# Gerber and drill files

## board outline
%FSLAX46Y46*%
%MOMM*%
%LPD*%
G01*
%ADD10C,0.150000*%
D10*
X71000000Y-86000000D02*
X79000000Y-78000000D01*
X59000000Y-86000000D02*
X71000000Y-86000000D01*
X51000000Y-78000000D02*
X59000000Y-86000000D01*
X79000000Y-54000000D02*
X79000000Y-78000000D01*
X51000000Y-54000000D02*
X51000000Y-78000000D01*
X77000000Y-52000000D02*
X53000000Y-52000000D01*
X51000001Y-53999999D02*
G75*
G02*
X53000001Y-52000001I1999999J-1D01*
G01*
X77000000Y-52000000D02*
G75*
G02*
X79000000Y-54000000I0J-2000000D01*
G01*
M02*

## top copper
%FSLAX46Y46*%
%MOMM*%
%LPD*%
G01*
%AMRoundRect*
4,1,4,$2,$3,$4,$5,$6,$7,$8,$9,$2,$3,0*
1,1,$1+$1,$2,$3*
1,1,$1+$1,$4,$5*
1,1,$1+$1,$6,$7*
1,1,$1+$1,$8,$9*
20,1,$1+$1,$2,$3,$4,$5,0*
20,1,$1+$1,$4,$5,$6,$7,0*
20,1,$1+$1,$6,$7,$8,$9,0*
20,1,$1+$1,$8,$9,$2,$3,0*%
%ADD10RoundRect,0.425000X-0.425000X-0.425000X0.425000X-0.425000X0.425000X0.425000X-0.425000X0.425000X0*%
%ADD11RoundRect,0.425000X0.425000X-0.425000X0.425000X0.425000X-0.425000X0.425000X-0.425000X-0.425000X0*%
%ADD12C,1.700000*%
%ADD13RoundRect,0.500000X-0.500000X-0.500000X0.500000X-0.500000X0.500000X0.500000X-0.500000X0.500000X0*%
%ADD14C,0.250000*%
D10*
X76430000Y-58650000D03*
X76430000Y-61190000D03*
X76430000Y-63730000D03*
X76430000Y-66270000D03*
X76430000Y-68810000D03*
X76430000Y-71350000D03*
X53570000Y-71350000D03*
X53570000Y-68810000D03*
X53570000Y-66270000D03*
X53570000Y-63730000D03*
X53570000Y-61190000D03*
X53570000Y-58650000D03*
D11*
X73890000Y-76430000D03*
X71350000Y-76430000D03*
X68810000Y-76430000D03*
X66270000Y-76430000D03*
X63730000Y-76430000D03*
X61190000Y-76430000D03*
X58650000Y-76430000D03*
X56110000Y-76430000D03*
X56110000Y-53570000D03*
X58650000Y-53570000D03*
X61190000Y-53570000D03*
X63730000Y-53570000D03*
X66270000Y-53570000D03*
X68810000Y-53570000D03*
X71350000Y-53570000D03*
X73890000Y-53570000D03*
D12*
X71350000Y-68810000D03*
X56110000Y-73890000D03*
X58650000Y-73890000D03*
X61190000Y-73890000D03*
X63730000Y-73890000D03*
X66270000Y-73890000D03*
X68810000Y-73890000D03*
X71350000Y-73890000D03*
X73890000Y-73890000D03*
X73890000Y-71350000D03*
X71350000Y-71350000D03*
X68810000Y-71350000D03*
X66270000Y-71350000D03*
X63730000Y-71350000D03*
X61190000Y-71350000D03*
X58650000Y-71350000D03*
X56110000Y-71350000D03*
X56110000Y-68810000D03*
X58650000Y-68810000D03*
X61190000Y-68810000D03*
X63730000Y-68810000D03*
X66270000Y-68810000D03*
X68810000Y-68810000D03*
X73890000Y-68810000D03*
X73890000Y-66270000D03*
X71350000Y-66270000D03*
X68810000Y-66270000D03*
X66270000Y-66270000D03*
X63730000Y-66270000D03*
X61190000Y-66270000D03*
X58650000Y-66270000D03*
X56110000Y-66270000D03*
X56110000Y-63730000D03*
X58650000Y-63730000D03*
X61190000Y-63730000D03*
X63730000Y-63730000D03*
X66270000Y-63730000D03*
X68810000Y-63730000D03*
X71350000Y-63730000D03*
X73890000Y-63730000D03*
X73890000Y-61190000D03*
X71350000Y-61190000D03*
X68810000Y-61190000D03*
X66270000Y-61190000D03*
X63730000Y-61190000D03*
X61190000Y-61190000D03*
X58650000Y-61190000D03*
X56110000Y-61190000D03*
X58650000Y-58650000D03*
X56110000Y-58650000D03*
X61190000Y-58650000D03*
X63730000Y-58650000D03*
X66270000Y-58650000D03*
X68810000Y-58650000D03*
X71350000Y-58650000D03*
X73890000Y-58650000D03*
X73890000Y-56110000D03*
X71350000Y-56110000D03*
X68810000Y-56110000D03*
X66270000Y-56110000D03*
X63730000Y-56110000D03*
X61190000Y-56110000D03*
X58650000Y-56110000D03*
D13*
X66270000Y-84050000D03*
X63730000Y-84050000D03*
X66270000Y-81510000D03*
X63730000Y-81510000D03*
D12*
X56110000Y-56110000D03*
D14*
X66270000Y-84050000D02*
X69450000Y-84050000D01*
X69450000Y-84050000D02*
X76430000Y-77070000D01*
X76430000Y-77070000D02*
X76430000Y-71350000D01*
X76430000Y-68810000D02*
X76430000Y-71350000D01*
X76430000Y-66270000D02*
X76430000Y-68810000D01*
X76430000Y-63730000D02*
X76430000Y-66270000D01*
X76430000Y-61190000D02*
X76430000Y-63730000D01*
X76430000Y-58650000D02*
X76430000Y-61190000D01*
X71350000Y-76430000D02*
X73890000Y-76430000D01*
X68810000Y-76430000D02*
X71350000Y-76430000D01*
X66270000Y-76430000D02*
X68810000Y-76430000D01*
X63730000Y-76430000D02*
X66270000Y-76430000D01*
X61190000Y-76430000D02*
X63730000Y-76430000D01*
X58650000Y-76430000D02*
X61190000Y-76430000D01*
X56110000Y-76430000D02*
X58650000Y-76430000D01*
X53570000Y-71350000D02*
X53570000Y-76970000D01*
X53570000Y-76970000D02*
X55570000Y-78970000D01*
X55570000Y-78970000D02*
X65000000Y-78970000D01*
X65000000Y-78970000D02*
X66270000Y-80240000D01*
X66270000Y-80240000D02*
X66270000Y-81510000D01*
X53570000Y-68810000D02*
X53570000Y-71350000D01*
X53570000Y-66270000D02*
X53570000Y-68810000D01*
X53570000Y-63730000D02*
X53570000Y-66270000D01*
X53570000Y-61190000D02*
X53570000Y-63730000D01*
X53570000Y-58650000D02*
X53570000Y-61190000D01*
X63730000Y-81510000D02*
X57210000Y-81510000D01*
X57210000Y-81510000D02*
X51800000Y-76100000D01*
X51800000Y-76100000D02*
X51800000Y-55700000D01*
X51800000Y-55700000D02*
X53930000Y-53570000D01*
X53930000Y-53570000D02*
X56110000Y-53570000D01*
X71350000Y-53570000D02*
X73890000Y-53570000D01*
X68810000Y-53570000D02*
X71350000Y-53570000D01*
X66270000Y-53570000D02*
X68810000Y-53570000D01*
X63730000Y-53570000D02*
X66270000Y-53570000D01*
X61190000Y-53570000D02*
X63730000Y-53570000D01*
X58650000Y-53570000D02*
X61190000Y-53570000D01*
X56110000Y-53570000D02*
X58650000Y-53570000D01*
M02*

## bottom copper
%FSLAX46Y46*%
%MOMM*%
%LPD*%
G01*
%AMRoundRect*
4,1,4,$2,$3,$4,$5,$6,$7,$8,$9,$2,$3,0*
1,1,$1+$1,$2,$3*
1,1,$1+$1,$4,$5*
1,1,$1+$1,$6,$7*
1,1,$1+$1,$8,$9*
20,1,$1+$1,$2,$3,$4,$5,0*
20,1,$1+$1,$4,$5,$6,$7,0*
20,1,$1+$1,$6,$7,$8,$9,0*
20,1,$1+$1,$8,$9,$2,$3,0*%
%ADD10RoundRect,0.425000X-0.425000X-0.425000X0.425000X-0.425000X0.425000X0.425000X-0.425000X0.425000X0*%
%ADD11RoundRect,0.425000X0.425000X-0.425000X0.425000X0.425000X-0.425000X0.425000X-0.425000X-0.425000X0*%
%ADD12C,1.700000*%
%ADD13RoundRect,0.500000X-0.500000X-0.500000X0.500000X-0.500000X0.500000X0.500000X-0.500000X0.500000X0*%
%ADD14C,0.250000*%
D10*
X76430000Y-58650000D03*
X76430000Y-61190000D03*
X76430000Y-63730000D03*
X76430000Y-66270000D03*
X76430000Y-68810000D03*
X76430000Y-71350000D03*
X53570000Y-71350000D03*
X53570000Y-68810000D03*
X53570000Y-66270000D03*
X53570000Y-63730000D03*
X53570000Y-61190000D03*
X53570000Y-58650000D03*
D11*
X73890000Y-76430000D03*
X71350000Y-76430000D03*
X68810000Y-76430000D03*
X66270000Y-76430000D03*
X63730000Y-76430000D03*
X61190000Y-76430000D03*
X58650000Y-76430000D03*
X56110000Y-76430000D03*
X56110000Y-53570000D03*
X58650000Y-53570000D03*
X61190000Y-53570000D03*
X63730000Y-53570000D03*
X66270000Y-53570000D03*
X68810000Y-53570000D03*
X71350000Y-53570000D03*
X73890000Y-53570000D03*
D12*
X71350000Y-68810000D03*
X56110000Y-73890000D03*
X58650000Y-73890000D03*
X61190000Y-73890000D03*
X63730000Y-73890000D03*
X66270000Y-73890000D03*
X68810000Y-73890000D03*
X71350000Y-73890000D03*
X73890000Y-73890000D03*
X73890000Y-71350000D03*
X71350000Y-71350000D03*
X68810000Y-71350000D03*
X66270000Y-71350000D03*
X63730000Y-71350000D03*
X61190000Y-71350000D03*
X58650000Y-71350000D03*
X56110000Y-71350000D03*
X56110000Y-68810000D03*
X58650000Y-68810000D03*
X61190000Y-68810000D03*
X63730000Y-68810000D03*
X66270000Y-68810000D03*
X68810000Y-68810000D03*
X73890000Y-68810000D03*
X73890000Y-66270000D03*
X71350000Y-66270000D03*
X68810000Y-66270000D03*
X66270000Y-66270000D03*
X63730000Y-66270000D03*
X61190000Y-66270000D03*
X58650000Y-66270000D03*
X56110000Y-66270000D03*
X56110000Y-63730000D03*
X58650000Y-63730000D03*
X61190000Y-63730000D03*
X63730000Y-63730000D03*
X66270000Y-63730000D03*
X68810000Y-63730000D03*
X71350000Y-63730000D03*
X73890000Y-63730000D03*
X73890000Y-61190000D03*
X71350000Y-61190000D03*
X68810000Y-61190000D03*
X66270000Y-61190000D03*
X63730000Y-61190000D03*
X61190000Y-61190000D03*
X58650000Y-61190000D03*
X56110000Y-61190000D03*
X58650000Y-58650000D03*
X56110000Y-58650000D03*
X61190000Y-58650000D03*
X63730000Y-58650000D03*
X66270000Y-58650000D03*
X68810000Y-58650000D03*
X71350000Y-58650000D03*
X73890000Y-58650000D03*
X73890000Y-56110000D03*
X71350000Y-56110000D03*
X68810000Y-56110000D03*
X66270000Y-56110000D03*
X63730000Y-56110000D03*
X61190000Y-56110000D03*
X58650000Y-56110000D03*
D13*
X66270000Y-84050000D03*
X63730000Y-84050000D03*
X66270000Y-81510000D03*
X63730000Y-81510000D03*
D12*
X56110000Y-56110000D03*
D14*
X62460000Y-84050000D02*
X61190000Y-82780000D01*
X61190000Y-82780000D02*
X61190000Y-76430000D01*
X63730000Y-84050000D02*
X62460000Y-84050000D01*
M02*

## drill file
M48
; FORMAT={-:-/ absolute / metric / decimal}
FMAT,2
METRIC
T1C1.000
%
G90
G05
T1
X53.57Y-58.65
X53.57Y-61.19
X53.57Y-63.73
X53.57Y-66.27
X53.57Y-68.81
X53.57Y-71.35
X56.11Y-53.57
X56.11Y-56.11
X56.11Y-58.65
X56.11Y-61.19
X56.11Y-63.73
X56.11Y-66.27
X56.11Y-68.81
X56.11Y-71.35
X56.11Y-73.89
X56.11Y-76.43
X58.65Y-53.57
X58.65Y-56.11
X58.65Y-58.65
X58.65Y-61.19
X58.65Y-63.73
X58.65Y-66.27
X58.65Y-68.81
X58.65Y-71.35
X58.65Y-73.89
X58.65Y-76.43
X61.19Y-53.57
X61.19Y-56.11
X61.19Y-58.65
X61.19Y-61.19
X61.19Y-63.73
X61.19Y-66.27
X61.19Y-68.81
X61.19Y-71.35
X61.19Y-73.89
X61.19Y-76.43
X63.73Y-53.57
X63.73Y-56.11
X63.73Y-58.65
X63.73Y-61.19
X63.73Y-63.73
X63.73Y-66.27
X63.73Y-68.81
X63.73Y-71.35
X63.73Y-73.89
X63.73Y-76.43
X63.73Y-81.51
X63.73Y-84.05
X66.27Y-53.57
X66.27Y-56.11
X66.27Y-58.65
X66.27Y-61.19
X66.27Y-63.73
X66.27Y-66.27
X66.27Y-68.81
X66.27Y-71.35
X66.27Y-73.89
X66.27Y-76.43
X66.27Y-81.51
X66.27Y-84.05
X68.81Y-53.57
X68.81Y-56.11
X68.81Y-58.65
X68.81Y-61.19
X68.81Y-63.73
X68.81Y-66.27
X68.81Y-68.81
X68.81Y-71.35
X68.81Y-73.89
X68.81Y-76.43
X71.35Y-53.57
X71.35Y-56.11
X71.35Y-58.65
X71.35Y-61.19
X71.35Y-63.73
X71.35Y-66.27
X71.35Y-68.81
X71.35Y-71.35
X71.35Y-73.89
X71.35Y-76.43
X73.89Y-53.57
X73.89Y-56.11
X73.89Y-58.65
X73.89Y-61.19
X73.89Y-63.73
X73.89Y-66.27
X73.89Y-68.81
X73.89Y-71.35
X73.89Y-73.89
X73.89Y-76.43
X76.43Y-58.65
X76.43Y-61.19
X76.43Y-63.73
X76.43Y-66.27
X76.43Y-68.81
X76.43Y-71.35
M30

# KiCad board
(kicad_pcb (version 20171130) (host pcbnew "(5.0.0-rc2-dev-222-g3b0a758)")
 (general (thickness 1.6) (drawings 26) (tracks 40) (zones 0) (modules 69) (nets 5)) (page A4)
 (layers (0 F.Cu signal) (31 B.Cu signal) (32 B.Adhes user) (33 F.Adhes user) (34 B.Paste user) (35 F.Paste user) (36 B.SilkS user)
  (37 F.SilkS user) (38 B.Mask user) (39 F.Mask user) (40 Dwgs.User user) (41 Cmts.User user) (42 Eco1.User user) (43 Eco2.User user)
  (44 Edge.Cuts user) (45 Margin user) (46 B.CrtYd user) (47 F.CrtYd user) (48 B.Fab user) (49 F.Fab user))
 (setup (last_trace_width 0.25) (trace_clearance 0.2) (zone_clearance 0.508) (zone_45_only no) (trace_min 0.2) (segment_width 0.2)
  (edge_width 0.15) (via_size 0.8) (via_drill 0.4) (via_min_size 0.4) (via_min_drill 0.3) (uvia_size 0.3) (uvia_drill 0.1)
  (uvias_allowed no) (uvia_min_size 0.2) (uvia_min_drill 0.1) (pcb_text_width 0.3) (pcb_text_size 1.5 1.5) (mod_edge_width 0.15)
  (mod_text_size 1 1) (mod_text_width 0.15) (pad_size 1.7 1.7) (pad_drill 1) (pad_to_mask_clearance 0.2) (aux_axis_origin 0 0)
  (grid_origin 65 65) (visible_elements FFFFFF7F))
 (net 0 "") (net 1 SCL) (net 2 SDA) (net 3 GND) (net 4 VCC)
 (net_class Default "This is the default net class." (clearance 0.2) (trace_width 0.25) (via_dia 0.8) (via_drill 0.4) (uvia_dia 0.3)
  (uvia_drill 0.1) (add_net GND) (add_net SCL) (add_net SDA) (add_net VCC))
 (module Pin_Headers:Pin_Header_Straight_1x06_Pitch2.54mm (layer F.Cu) (at 76.43 58.65)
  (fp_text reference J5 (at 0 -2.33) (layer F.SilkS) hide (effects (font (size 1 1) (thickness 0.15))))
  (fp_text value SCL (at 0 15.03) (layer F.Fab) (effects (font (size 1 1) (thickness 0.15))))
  (pad 1 thru_hole roundrect (at 0 0) (size 1.7 1.7) (drill 1) (layers *.Cu *.Mask) (roundrect_rratio 0.25) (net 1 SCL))
  (pad 2 thru_hole roundrect (at 0 2.54) (size 1.7 1.7) (drill 1) (layers *.Cu *.Mask) (roundrect_rratio 0.25) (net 1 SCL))
  (pad 3 thru_hole roundrect (at 0 5.08) (size 1.7 1.7) (drill 1) (layers *.Cu *.Mask) (roundrect_rratio 0.25) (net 1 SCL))
  (pad 4 thru_hole roundrect (at 0 7.62) (size 1.7 1.7) (drill 1) (layers *.Cu *.Mask) (roundrect_rratio 0.25) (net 1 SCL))
  (pad 5 thru_hole roundrect (at 0 10.16) (size 1.7 1.7) (drill 1) (layers *.Cu *.Mask) (roundrect_rratio 0.25) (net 1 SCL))
  (pad 6 thru_hole roundrect (at 0 12.7) (size 1.7 1.7) (drill 1) (layers *.Cu *.Mask) (roundrect_rratio 0.25) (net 1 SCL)))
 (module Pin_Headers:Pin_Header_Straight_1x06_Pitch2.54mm (layer F.Cu) (at 53.57 58.65)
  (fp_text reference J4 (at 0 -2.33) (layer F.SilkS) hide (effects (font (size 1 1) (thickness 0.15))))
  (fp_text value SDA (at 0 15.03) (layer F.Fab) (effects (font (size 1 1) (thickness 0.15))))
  (pad 6 thru_hole roundrect (at 0 12.7) (size 1.7 1.7) (drill 1) (layers *.Cu *.Mask) (roundrect_rratio 0.25) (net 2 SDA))
  (pad 5 thru_hole roundrect (at 0 10.16) (size 1.7 1.7) (drill 1) (layers *.Cu *.Mask) (roundrect_rratio 0.25) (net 2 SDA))
  (pad 4 thru_hole roundrect (at 0 7.62) (size 1.7 1.7) (drill 1) (layers *.Cu *.Mask) (roundrect_rratio 0.25) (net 2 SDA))
  (pad 3 thru_hole roundrect (at 0 5.08) (size 1.7 1.7) (drill 1) (layers *.Cu *.Mask) (roundrect_rratio 0.25) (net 2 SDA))
  (pad 2 thru_hole roundrect (at 0 2.54) (size 1.7 1.7) (drill 1) (layers *.Cu *.Mask) (roundrect_rratio 0.25) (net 2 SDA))
  (pad 1 thru_hole roundrect (at 0 0) (size 1.7 1.7) (drill 1) (layers *.Cu *.Mask) (roundrect_rratio 0.25) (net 2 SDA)))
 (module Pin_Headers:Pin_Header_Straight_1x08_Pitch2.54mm (layer F.Cu) (at 56.11 76.43 90)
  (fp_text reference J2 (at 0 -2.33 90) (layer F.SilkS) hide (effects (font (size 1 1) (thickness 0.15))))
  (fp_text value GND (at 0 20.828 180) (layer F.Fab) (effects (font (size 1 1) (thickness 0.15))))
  (pad 8 thru_hole roundrect (at 0 17.78 90) (size 1.7 1.7) (drill 1) (layers *.Cu *.Mask) (roundrect_rratio 0.25) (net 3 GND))
  (pad 7 thru_hole roundrect (at 0 15.24 90) (size 1.7 1.7) (drill 1) (layers *.Cu *.Mask) (roundrect_rratio 0.25) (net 3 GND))
  (pad 6 thru_hole roundrect (at 0 12.7 90) (size 1.7 1.7) (drill 1) (layers *.Cu *.Mask) (roundrect_rratio 0.25) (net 3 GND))
  (pad 5 thru_hole roundrect (at 0 10.16 90) (size 1.7 1.7) (drill 1) (layers *.Cu *.Mask) (roundrect_rratio 0.25) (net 3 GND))
  (pad 4 thru_hole roundrect (at 0 7.62 90) (size 1.7 1.7) (drill 1) (layers *.Cu *.Mask) (roundrect_rratio 0.25) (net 3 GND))
  (pad 3 thru_hole roundrect (at 0 5.08 90) (size 1.7 1.7) (drill 1) (layers *.Cu *.Mask) (roundrect_rratio 0.25) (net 3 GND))
  (pad 2 thru_hole roundrect (at 0 2.54 90) (size 1.7 1.7) (drill 1) (layers *.Cu *.Mask) (roundrect_rratio 0.25) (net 3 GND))
  (pad 1 thru_hole roundrect (at 0 0 90) (size 1.7 1.7) (drill 1) (layers *.Cu *.Mask) (roundrect_rratio 0.25) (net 3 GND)))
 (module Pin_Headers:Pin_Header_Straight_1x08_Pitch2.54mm (layer F.Cu) (at 56.11 53.57 90)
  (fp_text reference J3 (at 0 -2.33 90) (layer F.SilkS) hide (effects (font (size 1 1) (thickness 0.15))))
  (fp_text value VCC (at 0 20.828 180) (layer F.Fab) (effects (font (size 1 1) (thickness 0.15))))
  (pad 1 thru_hole roundrect (at 0 0 90) (size 1.7 1.7) (drill 1) (layers *.Cu *.Mask) (roundrect_rratio 0.25) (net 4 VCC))
  (pad 2 thru_hole roundrect (at 0 2.54 90) (size 1.7 1.7) (drill 1) (layers *.Cu *.Mask) (roundrect_rratio 0.25) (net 4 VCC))
  (pad 3 thru_hole roundrect (at 0 5.08 90) (size 1.7 1.7) (drill 1) (layers *.Cu *.Mask) (roundrect_rratio 0.25) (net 4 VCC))
  (pad 4 thru_hole roundrect (at 0 7.62 90) (size 1.7 1.7) (drill 1) (layers *.Cu *.Mask) (roundrect_rratio 0.25) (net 4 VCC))
  (pad 5 thru_hole roundrect (at 0 10.16 90) (size 1.7 1.7) (drill 1) (layers *.Cu *.Mask) (roundrect_rratio 0.25) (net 4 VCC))
  (pad 6 thru_hole roundrect (at 0 12.7 90) (size 1.7 1.7) (drill 1) (layers *.Cu *.Mask) (roundrect_rratio 0.25) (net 4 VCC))
  (pad 7 thru_hole roundrect (at 0 15.24 90) (size 1.7 1.7) (drill 1) (layers *.Cu *.Mask) (roundrect_rratio 0.25) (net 4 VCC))
  (pad 8 thru_hole roundrect (at 0 17.78 90) (size 1.7 1.7) (drill 1) (layers *.Cu *.Mask) (roundrect_rratio 0.25) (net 4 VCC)))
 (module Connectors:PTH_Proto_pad (layer F.Cu) (at 71.35 68.81)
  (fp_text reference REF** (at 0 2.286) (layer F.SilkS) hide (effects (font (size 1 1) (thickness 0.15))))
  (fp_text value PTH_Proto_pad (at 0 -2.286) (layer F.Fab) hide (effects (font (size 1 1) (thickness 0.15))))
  (pad 1 thru_hole circle (at 0 0) (size 1.7 1.7) (drill 1) (layers *.Cu *.Mask F.SilkS)))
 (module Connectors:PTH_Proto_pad (layer F.Cu) (at 56.11 73.89)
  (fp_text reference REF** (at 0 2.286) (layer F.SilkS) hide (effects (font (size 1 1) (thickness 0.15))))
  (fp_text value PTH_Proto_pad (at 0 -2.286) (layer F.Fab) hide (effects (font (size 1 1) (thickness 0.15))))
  (pad 1 thru_hole circle (at 0 0) (size 1.7 1.7) (drill 1) (layers *.Cu *.Mask F.SilkS)))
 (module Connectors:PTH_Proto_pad (layer F.Cu) (at 58.65 73.89)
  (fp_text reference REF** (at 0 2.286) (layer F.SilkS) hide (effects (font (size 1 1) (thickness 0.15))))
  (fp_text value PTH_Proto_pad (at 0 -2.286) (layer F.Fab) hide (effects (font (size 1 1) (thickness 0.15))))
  (pad 1 thru_hole circle (at 0 0) (size 1.7 1.7) (drill 1) (layers *.Cu *.Mask F.SilkS)))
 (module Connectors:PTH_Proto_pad (layer F.Cu) (at 61.19 73.89)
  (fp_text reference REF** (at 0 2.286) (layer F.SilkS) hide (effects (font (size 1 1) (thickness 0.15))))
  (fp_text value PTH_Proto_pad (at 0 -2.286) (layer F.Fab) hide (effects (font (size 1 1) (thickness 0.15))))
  (pad 1 thru_hole circle (at 0 0) (size 1.7 1.7) (drill 1) (layers *.Cu *.Mask F.SilkS)))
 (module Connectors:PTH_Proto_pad (layer F.Cu) (at 63.73 73.89)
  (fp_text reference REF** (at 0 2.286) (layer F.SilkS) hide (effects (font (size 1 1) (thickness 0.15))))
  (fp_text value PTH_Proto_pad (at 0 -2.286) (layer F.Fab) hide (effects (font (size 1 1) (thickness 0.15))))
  (pad 1 thru_hole circle (at 0 0) (size 1.7 1.7) (drill 1) (layers *.Cu *.Mask F.SilkS)))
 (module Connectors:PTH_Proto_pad (layer F.Cu) (at 66.27 73.89)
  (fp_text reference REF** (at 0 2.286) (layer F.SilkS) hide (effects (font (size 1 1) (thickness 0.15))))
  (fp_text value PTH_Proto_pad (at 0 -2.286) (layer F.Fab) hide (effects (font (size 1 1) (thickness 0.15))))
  (pad 1 thru_hole circle (at 0 0) (size 1.7 1.7) (drill 1) (layers *.Cu *.Mask F.SilkS)))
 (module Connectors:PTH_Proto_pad (layer F.Cu) (at 68.81 73.89)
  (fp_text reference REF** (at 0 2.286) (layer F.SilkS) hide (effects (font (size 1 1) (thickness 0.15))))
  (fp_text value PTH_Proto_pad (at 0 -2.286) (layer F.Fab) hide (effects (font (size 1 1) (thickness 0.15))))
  (pad 1 thru_hole circle (at 0 0) (size 1.7 1.7) (drill 1) (layers *.Cu *.Mask F.SilkS)))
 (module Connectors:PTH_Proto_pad (layer F.Cu) (at 71.35 73.89)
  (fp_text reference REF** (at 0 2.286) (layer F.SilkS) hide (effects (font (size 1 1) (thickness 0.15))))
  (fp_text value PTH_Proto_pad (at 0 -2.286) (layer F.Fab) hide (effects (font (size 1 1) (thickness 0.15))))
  (pad 1 thru_hole circle (at 0 0) (size 1.7 1.7) (drill 1) (layers *.Cu *.Mask F.SilkS)))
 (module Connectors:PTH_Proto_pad (layer F.Cu) (at 73.89 73.89)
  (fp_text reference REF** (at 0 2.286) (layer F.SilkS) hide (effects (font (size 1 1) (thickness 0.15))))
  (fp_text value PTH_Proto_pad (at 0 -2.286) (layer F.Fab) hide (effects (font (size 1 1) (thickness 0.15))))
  (pad 1 thru_hole circle (at 0 0) (size 1.7 1.7) (drill 1) (layers *.Cu *.Mask F.SilkS)))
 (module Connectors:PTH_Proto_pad (layer F.Cu) (at 73.89 71.35)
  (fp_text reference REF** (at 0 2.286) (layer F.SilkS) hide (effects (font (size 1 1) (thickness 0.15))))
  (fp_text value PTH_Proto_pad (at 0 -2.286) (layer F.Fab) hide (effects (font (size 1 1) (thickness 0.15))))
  (pad 1 thru_hole circle (at 0 0) (size 1.7 1.7) (drill 1) (layers *.Cu *.Mask F.SilkS)))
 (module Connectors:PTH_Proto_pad (layer F.Cu) (at 71.35 71.35)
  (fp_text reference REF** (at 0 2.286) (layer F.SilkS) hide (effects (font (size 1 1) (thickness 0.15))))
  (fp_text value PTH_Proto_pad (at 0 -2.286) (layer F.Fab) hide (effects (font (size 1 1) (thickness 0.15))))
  (pad 1 thru_hole circle (at 0 0) (size 1.7 1.7) (drill 1) (layers *.Cu *.Mask F.SilkS)))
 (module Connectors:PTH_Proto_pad (layer F.Cu) (at 68.81 71.35)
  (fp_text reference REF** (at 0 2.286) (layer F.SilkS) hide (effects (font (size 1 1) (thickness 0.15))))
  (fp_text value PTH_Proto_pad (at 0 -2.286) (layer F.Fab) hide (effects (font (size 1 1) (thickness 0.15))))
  (pad 1 thru_hole circle (at 0 0) (size 1.7 1.7) (drill 1) (layers *.Cu *.Mask F.SilkS)))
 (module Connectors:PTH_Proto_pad (layer F.Cu) (at 66.27 71.35)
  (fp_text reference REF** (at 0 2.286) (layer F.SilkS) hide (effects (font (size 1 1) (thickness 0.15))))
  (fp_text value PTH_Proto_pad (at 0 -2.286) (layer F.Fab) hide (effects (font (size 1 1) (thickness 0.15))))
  (pad 1 thru_hole circle (at 0 0) (size 1.7 1.7) (drill 1) (layers *.Cu *.Mask F.SilkS)))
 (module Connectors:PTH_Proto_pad (layer F.Cu) (at 63.73 71.35)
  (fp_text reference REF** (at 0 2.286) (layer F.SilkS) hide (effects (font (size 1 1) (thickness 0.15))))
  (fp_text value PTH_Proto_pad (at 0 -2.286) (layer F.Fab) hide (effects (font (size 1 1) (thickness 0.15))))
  (pad 1 thru_hole circle (at 0 0) (size 1.7 1.7) (drill 1) (layers *.Cu *.Mask F.SilkS)))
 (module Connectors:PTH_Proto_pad (layer F.Cu) (at 61.19 71.35)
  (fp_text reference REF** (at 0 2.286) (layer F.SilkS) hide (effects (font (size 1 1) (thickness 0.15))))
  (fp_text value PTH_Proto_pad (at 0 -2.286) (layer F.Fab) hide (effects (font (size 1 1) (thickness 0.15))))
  (pad 1 thru_hole circle (at 0 0) (size 1.7 1.7) (drill 1) (layers *.Cu *.Mask F.SilkS)))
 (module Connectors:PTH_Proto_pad (layer F.Cu) (at 58.65 71.35)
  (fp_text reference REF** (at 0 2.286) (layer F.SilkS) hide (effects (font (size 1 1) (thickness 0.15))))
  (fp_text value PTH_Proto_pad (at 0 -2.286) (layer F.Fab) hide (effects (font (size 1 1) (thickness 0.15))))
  (pad 1 thru_hole circle (at 0 0) (size 1.7 1.7) (drill 1) (layers *.Cu *.Mask F.SilkS)))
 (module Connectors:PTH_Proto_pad (layer F.Cu) (at 56.11 71.35)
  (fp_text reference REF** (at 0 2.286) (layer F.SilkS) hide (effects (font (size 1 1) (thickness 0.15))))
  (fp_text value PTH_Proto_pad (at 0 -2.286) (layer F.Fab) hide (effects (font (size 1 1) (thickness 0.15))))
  (pad 1 thru_hole circle (at 0 0) (size 1.7 1.7) (drill 1) (layers *.Cu *.Mask F.SilkS)))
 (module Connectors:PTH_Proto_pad (layer F.Cu) (at 56.11 68.81)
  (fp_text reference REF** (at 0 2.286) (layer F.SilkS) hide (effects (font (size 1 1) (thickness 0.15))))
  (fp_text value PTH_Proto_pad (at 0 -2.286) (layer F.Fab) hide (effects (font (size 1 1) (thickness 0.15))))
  (pad 1 thru_hole circle (at 0 0) (size 1.7 1.7) (drill 1) (layers *.Cu *.Mask F.SilkS)))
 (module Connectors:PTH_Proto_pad (layer F.Cu) (at 58.65 68.81)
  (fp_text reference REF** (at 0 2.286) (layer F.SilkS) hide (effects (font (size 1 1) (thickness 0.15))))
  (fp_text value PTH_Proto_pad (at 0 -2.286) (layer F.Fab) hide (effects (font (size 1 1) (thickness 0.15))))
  (pad 1 thru_hole circle (at 0 0) (size 1.7 1.7) (drill 1) (layers *.Cu *.Mask F.SilkS)))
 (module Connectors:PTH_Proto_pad (layer F.Cu) (at 61.19 68.81)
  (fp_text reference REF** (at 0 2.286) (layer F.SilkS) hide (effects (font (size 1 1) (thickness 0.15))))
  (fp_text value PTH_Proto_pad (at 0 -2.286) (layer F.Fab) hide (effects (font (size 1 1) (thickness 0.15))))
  (pad 1 thru_hole circle (at 0 0) (size 1.7 1.7) (drill 1) (layers *.Cu *.Mask F.SilkS)))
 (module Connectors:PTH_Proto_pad (layer F.Cu) (at 63.73 68.81)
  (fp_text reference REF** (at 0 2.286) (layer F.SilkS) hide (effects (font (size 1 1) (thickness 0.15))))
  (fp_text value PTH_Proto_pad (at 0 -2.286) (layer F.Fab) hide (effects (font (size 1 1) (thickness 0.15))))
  (pad 1 thru_hole circle (at 0 0) (size 1.7 1.7) (drill 1) (layers *.Cu *.Mask F.SilkS)))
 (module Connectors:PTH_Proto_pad (layer F.Cu) (at 66.27 68.81)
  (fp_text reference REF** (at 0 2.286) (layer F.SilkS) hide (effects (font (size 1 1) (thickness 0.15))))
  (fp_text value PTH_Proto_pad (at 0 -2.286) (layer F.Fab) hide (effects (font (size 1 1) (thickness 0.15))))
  (pad 1 thru_hole circle (at 0 0) (size 1.7 1.7) (drill 1) (layers *.Cu *.Mask F.SilkS)))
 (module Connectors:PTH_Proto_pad (layer F.Cu) (at 68.81 68.81)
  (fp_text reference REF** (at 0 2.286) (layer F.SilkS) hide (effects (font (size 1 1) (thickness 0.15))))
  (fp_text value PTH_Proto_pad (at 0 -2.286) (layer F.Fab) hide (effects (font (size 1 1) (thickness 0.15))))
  (pad 1 thru_hole circle (at 0 0) (size 1.7 1.7) (drill 1) (layers *.Cu *.Mask F.SilkS)))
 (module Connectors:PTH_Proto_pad (layer F.Cu) (at 73.89 68.81)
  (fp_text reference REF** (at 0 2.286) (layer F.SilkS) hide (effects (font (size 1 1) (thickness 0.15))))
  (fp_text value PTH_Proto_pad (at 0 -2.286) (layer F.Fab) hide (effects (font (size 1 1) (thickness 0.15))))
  (pad 1 thru_hole circle (at 0 0) (size 1.7 1.7) (drill 1) (layers *.Cu *.Mask F.SilkS)))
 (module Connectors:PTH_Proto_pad (layer F.Cu) (at 73.89 66.27)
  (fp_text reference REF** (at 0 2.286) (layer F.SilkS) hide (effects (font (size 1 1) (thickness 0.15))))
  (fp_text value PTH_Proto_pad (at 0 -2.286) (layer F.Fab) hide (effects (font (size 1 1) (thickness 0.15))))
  (pad 1 thru_hole circle (at 0 0) (size 1.7 1.7) (drill 1) (layers *.Cu *.Mask F.SilkS)))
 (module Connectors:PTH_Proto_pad (layer F.Cu) (at 71.35 66.27)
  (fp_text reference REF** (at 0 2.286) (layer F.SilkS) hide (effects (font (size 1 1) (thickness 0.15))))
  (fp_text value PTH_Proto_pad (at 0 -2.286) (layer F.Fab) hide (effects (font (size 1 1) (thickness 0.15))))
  (pad 1 thru_hole circle (at 0 0) (size 1.7 1.7) (drill 1) (layers *.Cu *.Mask F.SilkS)))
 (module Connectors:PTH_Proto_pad (layer F.Cu) (at 68.81 66.27)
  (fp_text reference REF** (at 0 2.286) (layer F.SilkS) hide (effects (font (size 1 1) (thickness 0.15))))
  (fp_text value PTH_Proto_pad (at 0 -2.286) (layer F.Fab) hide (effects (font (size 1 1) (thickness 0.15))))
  (pad 1 thru_hole circle (at 0 0) (size 1.7 1.7) (drill 1) (layers *.Cu *.Mask F.SilkS)))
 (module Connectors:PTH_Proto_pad (layer F.Cu) (at 66.27 66.27)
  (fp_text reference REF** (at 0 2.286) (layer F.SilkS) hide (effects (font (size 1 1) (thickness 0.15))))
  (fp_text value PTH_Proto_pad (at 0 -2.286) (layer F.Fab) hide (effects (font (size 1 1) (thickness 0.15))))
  (pad 1 thru_hole circle (at 0 0) (size 1.7 1.7) (drill 1) (layers *.Cu *.Mask F.SilkS)))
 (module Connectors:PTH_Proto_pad (layer F.Cu) (at 63.73 66.27)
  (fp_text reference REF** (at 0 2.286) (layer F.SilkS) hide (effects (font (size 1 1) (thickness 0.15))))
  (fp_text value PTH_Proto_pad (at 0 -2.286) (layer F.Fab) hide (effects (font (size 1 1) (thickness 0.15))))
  (pad 1 thru_hole circle (at 0 0) (size 1.7 1.7) (drill 1) (layers *.Cu *.Mask F.SilkS)))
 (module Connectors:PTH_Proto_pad (layer F.Cu) (at 61.19 66.27)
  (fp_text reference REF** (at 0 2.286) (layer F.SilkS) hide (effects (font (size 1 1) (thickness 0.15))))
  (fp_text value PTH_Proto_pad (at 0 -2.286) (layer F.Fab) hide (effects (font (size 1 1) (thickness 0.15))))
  (pad 1 thru_hole circle (at 0 0) (size 1.7 1.7) (drill 1) (layers *.Cu *.Mask F.SilkS)))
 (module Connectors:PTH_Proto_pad (layer F.Cu) (at 58.65 66.27)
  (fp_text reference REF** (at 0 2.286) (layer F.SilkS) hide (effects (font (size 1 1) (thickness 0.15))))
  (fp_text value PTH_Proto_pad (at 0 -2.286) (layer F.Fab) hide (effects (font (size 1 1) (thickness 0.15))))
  (pad 1 thru_hole circle (at 0 0) (size 1.7 1.7) (drill 1) (layers *.Cu *.Mask F.SilkS)))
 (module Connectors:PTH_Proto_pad (layer F.Cu) (at 56.11 66.27)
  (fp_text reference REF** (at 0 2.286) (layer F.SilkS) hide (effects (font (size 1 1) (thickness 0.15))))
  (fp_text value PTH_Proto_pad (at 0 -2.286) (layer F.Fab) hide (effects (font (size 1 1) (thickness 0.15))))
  (pad 1 thru_hole circle (at 0 0) (size 1.7 1.7) (drill 1) (layers *.Cu *.Mask F.SilkS)))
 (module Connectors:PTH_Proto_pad (layer F.Cu) (at 56.11 63.73)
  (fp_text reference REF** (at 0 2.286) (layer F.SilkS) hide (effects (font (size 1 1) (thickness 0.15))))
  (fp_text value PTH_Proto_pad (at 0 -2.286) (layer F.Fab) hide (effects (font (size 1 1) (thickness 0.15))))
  (pad 1 thru_hole circle (at 0 0) (size 1.7 1.7) (drill 1) (layers *.Cu *.Mask F.SilkS)))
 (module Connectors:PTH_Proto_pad (layer F.Cu) (at 58.65 63.73)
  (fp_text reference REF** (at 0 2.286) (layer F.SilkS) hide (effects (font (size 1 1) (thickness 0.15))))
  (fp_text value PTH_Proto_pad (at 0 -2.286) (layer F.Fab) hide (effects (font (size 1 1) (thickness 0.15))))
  (pad 1 thru_hole circle (at 0 0) (size 1.7 1.7) (drill 1) (layers *.Cu *.Mask F.SilkS)))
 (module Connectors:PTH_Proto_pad (layer F.Cu) (at 61.19 63.73)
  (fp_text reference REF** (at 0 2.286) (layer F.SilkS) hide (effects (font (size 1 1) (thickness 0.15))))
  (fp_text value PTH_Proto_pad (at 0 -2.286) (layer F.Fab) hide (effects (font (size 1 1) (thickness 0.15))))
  (pad 1 thru_hole circle (at 0 0) (size 1.7 1.7) (drill 1) (layers *.Cu *.Mask F.SilkS)))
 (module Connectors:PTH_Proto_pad (layer F.Cu) (at 63.73 63.73)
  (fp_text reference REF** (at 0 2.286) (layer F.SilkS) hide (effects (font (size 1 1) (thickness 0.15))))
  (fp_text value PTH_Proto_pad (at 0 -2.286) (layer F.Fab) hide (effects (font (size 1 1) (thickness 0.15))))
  (pad 1 thru_hole circle (at 0 0) (size 1.7 1.7) (drill 1) (layers *.Cu *.Mask F.SilkS)))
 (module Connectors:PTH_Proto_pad (layer F.Cu) (at 66.27 63.73)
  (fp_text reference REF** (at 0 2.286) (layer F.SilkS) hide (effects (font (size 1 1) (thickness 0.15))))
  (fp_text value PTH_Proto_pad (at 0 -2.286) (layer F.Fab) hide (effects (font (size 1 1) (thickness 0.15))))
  (pad 1 thru_hole circle (at 0 0) (size 1.7 1.7) (drill 1) (layers *.Cu *.Mask F.SilkS)))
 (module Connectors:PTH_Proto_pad (layer F.Cu) (at 68.81 63.73)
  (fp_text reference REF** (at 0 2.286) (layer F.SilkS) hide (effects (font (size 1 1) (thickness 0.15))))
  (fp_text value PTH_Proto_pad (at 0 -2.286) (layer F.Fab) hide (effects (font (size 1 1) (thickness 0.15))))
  (pad 1 thru_hole circle (at 0 0) (size 1.7 1.7) (drill 1) (layers *.Cu *.Mask F.SilkS)))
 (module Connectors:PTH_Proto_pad (layer F.Cu) (at 71.35 63.73)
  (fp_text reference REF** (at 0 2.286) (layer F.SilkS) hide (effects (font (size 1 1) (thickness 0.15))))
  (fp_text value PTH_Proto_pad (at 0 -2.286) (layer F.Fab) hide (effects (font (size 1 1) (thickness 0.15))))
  (pad 1 thru_hole circle (at 0 0) (size 1.7 1.7) (drill 1) (layers *.Cu *.Mask F.SilkS)))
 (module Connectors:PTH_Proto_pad (layer F.Cu) (at 73.89 63.73)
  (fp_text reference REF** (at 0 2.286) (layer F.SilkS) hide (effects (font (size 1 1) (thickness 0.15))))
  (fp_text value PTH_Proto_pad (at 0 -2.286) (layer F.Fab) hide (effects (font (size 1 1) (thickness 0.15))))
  (pad 1 thru_hole circle (at 0 0) (size 1.7 1.7) (drill 1) (layers *.Cu *.Mask F.SilkS)))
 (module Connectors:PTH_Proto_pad (layer F.Cu) (at 73.89 61.19)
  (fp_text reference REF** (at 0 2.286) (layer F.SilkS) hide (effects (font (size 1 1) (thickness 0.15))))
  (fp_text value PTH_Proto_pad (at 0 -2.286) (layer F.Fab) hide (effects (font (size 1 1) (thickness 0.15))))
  (pad 1 thru_hole circle (at 0 0) (size 1.7 1.7) (drill 1) (layers *.Cu *.Mask F.SilkS)))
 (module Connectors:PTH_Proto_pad (layer F.Cu) (at 71.35 61.19)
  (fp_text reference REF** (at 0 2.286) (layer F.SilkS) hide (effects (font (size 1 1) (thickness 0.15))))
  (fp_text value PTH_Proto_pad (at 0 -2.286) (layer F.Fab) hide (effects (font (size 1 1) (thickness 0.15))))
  (pad 1 thru_hole circle (at 0 0) (size 1.7 1.7) (drill 1) (layers *.Cu *.Mask F.SilkS)))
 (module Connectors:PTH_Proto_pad (layer F.Cu) (at 68.81 61.19)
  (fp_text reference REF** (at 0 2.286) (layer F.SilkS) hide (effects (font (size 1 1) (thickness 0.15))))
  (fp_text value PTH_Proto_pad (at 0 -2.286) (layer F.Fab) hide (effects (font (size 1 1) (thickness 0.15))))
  (pad 1 thru_hole circle (at 0 0) (size 1.7 1.7) (drill 1) (layers *.Cu *.Mask F.SilkS)))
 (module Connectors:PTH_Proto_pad (layer F.Cu) (at 66.27 61.19)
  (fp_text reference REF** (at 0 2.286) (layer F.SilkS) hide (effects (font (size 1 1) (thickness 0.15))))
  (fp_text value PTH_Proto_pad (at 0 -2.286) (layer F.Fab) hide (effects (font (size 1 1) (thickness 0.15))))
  (pad 1 thru_hole circle (at 0 0) (size 1.7 1.7) (drill 1) (layers *.Cu *.Mask F.SilkS)))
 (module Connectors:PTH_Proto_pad (layer F.Cu) (at 63.73 61.19)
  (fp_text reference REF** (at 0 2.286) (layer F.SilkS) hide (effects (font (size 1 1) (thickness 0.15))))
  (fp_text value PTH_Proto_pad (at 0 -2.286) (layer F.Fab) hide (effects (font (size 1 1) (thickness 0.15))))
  (pad 1 thru_hole circle (at 0 0) (size 1.7 1.7) (drill 1) (layers *.Cu *.Mask F.SilkS)))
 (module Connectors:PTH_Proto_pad (layer F.Cu) (at 61.19 61.19)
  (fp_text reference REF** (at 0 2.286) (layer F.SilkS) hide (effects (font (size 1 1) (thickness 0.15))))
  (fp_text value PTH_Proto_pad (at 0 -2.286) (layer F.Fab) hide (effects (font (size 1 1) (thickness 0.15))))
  (pad 1 thru_hole circle (at 0 0) (size 1.7 1.7) (drill 1) (layers *.Cu *.Mask F.SilkS)))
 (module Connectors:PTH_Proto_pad (layer F.Cu) (at 58.65 61.19)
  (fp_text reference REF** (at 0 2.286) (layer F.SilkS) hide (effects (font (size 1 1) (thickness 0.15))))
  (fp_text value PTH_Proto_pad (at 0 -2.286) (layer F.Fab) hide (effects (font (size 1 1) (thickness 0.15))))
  (pad 1 thru_hole circle (at 0 0) (size 1.7 1.7) (drill 1) (layers *.Cu *.Mask F.SilkS)))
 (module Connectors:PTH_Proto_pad (layer F.Cu) (at 56.11 61.19)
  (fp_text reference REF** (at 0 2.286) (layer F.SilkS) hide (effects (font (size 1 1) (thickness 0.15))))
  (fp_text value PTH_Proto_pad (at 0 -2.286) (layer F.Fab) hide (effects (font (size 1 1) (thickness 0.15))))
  (pad 1 thru_hole circle (at 0 0) (size 1.7 1.7) (drill 1) (layers *.Cu *.Mask F.SilkS)))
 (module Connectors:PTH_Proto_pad (layer F.Cu) (at 58.65 58.65)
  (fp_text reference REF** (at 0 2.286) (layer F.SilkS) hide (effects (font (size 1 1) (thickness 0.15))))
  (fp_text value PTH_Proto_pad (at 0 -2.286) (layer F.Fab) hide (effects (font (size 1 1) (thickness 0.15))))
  (pad 1 thru_hole circle (at 0 0) (size 1.7 1.7) (drill 1) (layers *.Cu *.Mask F.SilkS)))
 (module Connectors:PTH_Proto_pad (layer F.Cu) (at 56.11 58.65)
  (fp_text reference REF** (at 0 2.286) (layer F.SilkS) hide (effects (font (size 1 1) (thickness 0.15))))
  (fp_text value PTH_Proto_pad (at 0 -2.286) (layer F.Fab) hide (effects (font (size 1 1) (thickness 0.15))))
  (pad 1 thru_hole circle (at 0 0) (size 1.7 1.7) (drill 1) (layers *.Cu *.Mask F.SilkS)))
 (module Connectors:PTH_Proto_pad (layer F.Cu) (at 61.19 58.65)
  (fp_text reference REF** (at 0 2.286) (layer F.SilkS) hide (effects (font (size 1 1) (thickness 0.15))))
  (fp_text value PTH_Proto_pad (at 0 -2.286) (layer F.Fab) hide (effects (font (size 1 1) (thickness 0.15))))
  (pad 1 thru_hole circle (at 0 0) (size 1.7 1.7) (drill 1) (layers *.Cu *.Mask F.SilkS)))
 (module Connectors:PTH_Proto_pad (layer F.Cu) (at 63.73 58.65)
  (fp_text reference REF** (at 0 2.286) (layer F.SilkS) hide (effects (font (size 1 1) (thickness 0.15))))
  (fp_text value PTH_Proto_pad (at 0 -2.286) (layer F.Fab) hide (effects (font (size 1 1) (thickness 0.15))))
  (pad 1 thru_hole circle (at 0 0) (size 1.7 1.7) (drill 1) (layers *.Cu *.Mask F.SilkS)))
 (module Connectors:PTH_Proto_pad (layer F.Cu) (at 66.27 58.65)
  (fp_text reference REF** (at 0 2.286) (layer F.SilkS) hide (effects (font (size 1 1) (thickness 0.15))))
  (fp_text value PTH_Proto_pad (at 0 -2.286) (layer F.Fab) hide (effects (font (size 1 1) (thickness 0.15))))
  (pad 1 thru_hole circle (at 0 0) (size 1.7 1.7) (drill 1) (layers *.Cu *.Mask F.SilkS)))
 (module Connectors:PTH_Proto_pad (layer F.Cu) (at 68.81 58.65)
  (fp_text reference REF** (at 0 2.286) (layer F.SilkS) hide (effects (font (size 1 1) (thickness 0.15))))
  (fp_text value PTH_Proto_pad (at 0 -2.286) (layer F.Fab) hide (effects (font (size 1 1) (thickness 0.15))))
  (pad 1 thru_hole circle (at 0 0) (size 1.7 1.7) (drill 1) (layers *.Cu *.Mask F.SilkS)))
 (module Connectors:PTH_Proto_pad (layer F.Cu) (at 71.35 58.65)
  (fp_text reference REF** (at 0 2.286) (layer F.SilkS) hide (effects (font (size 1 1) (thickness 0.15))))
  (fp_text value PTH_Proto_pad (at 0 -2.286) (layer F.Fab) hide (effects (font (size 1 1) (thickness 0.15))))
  (pad 1 thru_hole circle (at 0 0) (size 1.7 1.7) (drill 1) (layers *.Cu *.Mask F.SilkS)))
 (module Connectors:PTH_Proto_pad (layer F.Cu) (at 73.89 58.65)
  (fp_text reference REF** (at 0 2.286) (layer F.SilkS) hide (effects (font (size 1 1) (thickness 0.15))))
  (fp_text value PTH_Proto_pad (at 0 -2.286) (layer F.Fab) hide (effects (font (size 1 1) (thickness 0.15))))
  (pad 1 thru_hole circle (at 0 0) (size 1.7 1.7) (drill 1) (layers *.Cu *.Mask F.SilkS)))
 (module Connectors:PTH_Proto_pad (layer F.Cu) (at 73.89 56.11)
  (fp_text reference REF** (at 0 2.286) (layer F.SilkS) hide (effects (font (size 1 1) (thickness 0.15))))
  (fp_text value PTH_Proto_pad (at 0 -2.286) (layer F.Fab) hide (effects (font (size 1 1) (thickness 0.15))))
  (pad 1 thru_hole circle (at 0 0) (size 1.7 1.7) (drill 1) (layers *.Cu *.Mask F.SilkS)))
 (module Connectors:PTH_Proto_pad (layer F.Cu) (at 71.35 56.11)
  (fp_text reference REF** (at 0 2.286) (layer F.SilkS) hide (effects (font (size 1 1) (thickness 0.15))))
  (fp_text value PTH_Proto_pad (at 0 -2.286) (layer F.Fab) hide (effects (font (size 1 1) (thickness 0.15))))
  (pad 1 thru_hole circle (at 0 0) (size 1.7 1.7) (drill 1) (layers *.Cu *.Mask F.SilkS)))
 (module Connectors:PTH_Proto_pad (layer F.Cu) (at 68.81 56.11)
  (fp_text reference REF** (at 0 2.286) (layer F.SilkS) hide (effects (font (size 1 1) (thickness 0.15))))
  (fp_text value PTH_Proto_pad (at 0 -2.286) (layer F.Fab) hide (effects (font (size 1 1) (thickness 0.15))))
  (pad 1 thru_hole circle (at 0 0) (size 1.7 1.7) (drill 1) (layers *.Cu *.Mask F.SilkS)))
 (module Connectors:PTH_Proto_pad (layer F.Cu) (at 66.27 56.11)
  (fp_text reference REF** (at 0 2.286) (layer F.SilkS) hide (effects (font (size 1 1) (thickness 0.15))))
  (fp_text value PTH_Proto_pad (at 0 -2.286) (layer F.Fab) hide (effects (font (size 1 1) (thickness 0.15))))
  (pad 1 thru_hole circle (at 0 0) (size 1.7 1.7) (drill 1) (layers *.Cu *.Mask F.SilkS)))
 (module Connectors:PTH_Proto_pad (layer F.Cu) (at 63.73 56.11)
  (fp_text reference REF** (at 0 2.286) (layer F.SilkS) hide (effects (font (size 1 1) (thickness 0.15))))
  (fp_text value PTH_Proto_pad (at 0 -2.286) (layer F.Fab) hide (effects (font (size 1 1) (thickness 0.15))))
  (pad 1 thru_hole circle (at 0 0) (size 1.7 1.7) (drill 1) (layers *.Cu *.Mask F.SilkS)))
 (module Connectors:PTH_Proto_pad (layer F.Cu) (at 61.19 56.11)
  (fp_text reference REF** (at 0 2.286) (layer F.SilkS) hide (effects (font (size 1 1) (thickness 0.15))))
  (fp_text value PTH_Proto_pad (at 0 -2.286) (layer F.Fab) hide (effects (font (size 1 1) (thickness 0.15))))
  (pad 1 thru_hole circle (at 0 0) (size 1.7 1.7) (drill 1) (layers *.Cu *.Mask F.SilkS)))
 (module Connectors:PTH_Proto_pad (layer F.Cu) (at 58.65 56.11)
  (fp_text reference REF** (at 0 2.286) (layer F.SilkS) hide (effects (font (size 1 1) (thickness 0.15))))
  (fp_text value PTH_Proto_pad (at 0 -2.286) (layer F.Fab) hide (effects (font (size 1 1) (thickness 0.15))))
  (pad 1 thru_hole circle (at 0 0) (size 1.7 1.7) (drill 1) (layers *.Cu *.Mask F.SilkS)))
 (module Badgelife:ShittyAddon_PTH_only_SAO (layer F.Cu) (at 63.73 81.51)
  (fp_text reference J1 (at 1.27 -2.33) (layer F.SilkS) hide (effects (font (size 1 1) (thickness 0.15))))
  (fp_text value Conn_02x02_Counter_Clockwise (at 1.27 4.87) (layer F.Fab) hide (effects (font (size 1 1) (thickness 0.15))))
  (pad 3 thru_hole roundrect (at 2.54 2.54) (size 2 2) (drill 1) (layers *.Cu *.Mask) (roundrect_rratio 0.25) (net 1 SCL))
  (pad 2 thru_hole roundrect (at 0 2.54) (size 2 2) (drill 1) (layers *.Cu *.Mask) (roundrect_rratio 0.25) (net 3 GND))
  (pad 4 thru_hole roundrect (at 2.54 0) (size 2 2) (drill 1) (layers *.Cu *.Mask) (roundrect_rratio 0.25) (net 2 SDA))
  (pad 1 thru_hole roundrect (at 0 0) (size 2 2) (drill 1) (layers *.Cu *.Mask) (roundrect_rratio 0.25) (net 4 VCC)))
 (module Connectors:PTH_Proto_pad (layer F.Cu) (at 56.11 56.11)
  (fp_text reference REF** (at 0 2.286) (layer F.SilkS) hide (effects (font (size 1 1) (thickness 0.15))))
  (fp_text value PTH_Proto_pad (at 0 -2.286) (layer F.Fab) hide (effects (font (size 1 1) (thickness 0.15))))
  (pad 1 thru_hole circle (at 0 0) (size 1.7 1.7) (drill 1) (layers *.Cu *.Mask F.SilkS)))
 (gr_line (start 71 86) (end 79 78) (layer Edge.Cuts) (width 0.15))
 (gr_line (start 59 86) (end 71 86) (layer Edge.Cuts) (width 0.15))
 (gr_line (start 51 78) (end 59 86) (layer Edge.Cuts) (width 0.15))
 (gr_line (start 79 54) (end 79 78) (layer Edge.Cuts) (width 0.15))
 (gr_line (start 51 54) (end 51 78) (layer Edge.Cuts) (width 0.15))
 (gr_line (start 77 52) (end 53 52) (layer Edge.Cuts) (width 0.15))
 (gr_arc (start 53 54) (end 53.000001 52.000001) (angle -90) (layer Edge.Cuts) (width 0.15))
 (gr_arc (start 77 54) (end 79 54) (angle -90) (layer Edge.Cuts) (width 0.15))
 (segment (start 66.27 84.05) (end 69.45 84.05) (width 0.25) (layer F.Cu) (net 1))
 (segment (start 69.45 84.05) (end 76.43 77.07) (width 0.25) (layer F.Cu) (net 1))
 (segment (start 76.43 77.07) (end 76.43 71.35) (width 0.25) (layer F.Cu) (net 1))
 (segment (start 76.43 68.81) (end 76.43 71.35) (width 0.25) (layer F.Cu) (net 1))
 (segment (start 76.43 66.27) (end 76.43 68.81) (width 0.25) (layer F.Cu) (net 1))
 (segment (start 76.43 63.73) (end 76.43 66.27) (width 0.25) (layer F.Cu) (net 1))
 (segment (start 76.43 61.19) (end 76.43 63.73) (width 0.25) (layer F.Cu) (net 1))
 (segment (start 76.43 58.65) (end 76.43 61.19) (width 0.25) (layer F.Cu) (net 1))
 (segment (start 62.46 84.05) (end 61.19 82.78) (width 0.25) (layer B.Cu) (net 3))
 (segment (start 61.19 82.78) (end 61.19 76.43) (width 0.25) (layer B.Cu) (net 3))
 (segment (start 63.73 84.05) (end 62.46 84.05) (width 0.25) (layer B.Cu) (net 3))
 (segment (start 71.35 76.43) (end 73.89 76.43) (width 0.25) (layer F.Cu) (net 3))
 (segment (start 68.81 76.43) (end 71.35 76.43) (width 0.25) (layer F.Cu) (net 3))
 (segment (start 66.27 76.43) (end 68.81 76.43) (width 0.25) (layer F.Cu) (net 3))
 (segment (start 63.73 76.43) (end 66.27 76.43) (width 0.25) (layer F.Cu) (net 3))
 (segment (start 61.19 76.43) (end 63.73 76.43) (width 0.25) (layer F.Cu) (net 3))
 (segment (start 58.65 76.43) (end 61.19 76.43) (width 0.25) (layer F.Cu) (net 3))
 (segment (start 56.11 76.43) (end 58.65 76.43) (width 0.25) (layer F.Cu) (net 3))
 (segment (start 53.57 71.35) (end 53.57 76.97) (width 0.25) (layer F.Cu) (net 2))
 (segment (start 53.57 76.97) (end 55.57 78.97) (width 0.25) (layer F.Cu) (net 2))
 (segment (start 55.57 78.97) (end 65 78.97) (width 0.25) (layer F.Cu) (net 2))
 (segment (start 65 78.97) (end 66.27 80.24) (width 0.25) (layer F.Cu) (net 2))
 (segment (start 66.27 80.24) (end 66.27 81.51) (width 0.25) (layer F.Cu) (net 2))
 (segment (start 53.57 68.81) (end 53.57 71.35) (width 0.25) (layer F.Cu) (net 2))
 (segment (start 53.57 66.27) (end 53.57 68.81) (width 0.25) (layer F.Cu) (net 2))
 (segment (start 53.57 63.73) (end 53.57 66.27) (width 0.25) (layer F.Cu) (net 2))
 (segment (start 53.57 61.19) (end 53.57 63.73) (width 0.25) (layer F.Cu) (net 2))
 (segment (start 53.57 58.65) (end 53.57 61.19) (width 0.25) (layer F.Cu) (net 2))
 (segment (start 63.73 81.51) (end 57.21 81.51) (width 0.25) (layer F.Cu) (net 4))
 (segment (start 57.21 81.51) (end 51.8 76.1) (width 0.25) (layer F.Cu) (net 4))
 (segment (start 51.8 76.1) (end 51.8 55.7) (width 0.25) (layer F.Cu) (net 4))
 (segment (start 51.8 55.7) (end 53.93 53.57) (width 0.25) (layer F.Cu) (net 4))
 (segment (start 53.93 53.57) (end 56.11 53.57) (width 0.25) (layer F.Cu) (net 4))
 (segment (start 71.35 53.57) (end 73.89 53.57) (width 0.25) (layer F.Cu) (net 4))
 (segment (start 68.81 53.57) (end 71.35 53.57) (width 0.25) (layer F.Cu) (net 4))
 (segment (start 66.27 53.57) (end 68.81 53.57) (width 0.25) (layer F.Cu) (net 4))
 (segment (start 63.73 53.57) (end 66.27 53.57) (width 0.25) (layer F.Cu) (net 4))
 (segment (start 61.19 53.57) (end 63.73 53.57) (width 0.25) (layer F.Cu) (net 4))
 (segment (start 58.65 53.57) (end 61.19 53.57) (width 0.25) (layer F.Cu) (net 4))
 (segment (start 56.11 53.57) (end 58.65 53.57) (width 0.25) (layer F.Cu) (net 4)))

